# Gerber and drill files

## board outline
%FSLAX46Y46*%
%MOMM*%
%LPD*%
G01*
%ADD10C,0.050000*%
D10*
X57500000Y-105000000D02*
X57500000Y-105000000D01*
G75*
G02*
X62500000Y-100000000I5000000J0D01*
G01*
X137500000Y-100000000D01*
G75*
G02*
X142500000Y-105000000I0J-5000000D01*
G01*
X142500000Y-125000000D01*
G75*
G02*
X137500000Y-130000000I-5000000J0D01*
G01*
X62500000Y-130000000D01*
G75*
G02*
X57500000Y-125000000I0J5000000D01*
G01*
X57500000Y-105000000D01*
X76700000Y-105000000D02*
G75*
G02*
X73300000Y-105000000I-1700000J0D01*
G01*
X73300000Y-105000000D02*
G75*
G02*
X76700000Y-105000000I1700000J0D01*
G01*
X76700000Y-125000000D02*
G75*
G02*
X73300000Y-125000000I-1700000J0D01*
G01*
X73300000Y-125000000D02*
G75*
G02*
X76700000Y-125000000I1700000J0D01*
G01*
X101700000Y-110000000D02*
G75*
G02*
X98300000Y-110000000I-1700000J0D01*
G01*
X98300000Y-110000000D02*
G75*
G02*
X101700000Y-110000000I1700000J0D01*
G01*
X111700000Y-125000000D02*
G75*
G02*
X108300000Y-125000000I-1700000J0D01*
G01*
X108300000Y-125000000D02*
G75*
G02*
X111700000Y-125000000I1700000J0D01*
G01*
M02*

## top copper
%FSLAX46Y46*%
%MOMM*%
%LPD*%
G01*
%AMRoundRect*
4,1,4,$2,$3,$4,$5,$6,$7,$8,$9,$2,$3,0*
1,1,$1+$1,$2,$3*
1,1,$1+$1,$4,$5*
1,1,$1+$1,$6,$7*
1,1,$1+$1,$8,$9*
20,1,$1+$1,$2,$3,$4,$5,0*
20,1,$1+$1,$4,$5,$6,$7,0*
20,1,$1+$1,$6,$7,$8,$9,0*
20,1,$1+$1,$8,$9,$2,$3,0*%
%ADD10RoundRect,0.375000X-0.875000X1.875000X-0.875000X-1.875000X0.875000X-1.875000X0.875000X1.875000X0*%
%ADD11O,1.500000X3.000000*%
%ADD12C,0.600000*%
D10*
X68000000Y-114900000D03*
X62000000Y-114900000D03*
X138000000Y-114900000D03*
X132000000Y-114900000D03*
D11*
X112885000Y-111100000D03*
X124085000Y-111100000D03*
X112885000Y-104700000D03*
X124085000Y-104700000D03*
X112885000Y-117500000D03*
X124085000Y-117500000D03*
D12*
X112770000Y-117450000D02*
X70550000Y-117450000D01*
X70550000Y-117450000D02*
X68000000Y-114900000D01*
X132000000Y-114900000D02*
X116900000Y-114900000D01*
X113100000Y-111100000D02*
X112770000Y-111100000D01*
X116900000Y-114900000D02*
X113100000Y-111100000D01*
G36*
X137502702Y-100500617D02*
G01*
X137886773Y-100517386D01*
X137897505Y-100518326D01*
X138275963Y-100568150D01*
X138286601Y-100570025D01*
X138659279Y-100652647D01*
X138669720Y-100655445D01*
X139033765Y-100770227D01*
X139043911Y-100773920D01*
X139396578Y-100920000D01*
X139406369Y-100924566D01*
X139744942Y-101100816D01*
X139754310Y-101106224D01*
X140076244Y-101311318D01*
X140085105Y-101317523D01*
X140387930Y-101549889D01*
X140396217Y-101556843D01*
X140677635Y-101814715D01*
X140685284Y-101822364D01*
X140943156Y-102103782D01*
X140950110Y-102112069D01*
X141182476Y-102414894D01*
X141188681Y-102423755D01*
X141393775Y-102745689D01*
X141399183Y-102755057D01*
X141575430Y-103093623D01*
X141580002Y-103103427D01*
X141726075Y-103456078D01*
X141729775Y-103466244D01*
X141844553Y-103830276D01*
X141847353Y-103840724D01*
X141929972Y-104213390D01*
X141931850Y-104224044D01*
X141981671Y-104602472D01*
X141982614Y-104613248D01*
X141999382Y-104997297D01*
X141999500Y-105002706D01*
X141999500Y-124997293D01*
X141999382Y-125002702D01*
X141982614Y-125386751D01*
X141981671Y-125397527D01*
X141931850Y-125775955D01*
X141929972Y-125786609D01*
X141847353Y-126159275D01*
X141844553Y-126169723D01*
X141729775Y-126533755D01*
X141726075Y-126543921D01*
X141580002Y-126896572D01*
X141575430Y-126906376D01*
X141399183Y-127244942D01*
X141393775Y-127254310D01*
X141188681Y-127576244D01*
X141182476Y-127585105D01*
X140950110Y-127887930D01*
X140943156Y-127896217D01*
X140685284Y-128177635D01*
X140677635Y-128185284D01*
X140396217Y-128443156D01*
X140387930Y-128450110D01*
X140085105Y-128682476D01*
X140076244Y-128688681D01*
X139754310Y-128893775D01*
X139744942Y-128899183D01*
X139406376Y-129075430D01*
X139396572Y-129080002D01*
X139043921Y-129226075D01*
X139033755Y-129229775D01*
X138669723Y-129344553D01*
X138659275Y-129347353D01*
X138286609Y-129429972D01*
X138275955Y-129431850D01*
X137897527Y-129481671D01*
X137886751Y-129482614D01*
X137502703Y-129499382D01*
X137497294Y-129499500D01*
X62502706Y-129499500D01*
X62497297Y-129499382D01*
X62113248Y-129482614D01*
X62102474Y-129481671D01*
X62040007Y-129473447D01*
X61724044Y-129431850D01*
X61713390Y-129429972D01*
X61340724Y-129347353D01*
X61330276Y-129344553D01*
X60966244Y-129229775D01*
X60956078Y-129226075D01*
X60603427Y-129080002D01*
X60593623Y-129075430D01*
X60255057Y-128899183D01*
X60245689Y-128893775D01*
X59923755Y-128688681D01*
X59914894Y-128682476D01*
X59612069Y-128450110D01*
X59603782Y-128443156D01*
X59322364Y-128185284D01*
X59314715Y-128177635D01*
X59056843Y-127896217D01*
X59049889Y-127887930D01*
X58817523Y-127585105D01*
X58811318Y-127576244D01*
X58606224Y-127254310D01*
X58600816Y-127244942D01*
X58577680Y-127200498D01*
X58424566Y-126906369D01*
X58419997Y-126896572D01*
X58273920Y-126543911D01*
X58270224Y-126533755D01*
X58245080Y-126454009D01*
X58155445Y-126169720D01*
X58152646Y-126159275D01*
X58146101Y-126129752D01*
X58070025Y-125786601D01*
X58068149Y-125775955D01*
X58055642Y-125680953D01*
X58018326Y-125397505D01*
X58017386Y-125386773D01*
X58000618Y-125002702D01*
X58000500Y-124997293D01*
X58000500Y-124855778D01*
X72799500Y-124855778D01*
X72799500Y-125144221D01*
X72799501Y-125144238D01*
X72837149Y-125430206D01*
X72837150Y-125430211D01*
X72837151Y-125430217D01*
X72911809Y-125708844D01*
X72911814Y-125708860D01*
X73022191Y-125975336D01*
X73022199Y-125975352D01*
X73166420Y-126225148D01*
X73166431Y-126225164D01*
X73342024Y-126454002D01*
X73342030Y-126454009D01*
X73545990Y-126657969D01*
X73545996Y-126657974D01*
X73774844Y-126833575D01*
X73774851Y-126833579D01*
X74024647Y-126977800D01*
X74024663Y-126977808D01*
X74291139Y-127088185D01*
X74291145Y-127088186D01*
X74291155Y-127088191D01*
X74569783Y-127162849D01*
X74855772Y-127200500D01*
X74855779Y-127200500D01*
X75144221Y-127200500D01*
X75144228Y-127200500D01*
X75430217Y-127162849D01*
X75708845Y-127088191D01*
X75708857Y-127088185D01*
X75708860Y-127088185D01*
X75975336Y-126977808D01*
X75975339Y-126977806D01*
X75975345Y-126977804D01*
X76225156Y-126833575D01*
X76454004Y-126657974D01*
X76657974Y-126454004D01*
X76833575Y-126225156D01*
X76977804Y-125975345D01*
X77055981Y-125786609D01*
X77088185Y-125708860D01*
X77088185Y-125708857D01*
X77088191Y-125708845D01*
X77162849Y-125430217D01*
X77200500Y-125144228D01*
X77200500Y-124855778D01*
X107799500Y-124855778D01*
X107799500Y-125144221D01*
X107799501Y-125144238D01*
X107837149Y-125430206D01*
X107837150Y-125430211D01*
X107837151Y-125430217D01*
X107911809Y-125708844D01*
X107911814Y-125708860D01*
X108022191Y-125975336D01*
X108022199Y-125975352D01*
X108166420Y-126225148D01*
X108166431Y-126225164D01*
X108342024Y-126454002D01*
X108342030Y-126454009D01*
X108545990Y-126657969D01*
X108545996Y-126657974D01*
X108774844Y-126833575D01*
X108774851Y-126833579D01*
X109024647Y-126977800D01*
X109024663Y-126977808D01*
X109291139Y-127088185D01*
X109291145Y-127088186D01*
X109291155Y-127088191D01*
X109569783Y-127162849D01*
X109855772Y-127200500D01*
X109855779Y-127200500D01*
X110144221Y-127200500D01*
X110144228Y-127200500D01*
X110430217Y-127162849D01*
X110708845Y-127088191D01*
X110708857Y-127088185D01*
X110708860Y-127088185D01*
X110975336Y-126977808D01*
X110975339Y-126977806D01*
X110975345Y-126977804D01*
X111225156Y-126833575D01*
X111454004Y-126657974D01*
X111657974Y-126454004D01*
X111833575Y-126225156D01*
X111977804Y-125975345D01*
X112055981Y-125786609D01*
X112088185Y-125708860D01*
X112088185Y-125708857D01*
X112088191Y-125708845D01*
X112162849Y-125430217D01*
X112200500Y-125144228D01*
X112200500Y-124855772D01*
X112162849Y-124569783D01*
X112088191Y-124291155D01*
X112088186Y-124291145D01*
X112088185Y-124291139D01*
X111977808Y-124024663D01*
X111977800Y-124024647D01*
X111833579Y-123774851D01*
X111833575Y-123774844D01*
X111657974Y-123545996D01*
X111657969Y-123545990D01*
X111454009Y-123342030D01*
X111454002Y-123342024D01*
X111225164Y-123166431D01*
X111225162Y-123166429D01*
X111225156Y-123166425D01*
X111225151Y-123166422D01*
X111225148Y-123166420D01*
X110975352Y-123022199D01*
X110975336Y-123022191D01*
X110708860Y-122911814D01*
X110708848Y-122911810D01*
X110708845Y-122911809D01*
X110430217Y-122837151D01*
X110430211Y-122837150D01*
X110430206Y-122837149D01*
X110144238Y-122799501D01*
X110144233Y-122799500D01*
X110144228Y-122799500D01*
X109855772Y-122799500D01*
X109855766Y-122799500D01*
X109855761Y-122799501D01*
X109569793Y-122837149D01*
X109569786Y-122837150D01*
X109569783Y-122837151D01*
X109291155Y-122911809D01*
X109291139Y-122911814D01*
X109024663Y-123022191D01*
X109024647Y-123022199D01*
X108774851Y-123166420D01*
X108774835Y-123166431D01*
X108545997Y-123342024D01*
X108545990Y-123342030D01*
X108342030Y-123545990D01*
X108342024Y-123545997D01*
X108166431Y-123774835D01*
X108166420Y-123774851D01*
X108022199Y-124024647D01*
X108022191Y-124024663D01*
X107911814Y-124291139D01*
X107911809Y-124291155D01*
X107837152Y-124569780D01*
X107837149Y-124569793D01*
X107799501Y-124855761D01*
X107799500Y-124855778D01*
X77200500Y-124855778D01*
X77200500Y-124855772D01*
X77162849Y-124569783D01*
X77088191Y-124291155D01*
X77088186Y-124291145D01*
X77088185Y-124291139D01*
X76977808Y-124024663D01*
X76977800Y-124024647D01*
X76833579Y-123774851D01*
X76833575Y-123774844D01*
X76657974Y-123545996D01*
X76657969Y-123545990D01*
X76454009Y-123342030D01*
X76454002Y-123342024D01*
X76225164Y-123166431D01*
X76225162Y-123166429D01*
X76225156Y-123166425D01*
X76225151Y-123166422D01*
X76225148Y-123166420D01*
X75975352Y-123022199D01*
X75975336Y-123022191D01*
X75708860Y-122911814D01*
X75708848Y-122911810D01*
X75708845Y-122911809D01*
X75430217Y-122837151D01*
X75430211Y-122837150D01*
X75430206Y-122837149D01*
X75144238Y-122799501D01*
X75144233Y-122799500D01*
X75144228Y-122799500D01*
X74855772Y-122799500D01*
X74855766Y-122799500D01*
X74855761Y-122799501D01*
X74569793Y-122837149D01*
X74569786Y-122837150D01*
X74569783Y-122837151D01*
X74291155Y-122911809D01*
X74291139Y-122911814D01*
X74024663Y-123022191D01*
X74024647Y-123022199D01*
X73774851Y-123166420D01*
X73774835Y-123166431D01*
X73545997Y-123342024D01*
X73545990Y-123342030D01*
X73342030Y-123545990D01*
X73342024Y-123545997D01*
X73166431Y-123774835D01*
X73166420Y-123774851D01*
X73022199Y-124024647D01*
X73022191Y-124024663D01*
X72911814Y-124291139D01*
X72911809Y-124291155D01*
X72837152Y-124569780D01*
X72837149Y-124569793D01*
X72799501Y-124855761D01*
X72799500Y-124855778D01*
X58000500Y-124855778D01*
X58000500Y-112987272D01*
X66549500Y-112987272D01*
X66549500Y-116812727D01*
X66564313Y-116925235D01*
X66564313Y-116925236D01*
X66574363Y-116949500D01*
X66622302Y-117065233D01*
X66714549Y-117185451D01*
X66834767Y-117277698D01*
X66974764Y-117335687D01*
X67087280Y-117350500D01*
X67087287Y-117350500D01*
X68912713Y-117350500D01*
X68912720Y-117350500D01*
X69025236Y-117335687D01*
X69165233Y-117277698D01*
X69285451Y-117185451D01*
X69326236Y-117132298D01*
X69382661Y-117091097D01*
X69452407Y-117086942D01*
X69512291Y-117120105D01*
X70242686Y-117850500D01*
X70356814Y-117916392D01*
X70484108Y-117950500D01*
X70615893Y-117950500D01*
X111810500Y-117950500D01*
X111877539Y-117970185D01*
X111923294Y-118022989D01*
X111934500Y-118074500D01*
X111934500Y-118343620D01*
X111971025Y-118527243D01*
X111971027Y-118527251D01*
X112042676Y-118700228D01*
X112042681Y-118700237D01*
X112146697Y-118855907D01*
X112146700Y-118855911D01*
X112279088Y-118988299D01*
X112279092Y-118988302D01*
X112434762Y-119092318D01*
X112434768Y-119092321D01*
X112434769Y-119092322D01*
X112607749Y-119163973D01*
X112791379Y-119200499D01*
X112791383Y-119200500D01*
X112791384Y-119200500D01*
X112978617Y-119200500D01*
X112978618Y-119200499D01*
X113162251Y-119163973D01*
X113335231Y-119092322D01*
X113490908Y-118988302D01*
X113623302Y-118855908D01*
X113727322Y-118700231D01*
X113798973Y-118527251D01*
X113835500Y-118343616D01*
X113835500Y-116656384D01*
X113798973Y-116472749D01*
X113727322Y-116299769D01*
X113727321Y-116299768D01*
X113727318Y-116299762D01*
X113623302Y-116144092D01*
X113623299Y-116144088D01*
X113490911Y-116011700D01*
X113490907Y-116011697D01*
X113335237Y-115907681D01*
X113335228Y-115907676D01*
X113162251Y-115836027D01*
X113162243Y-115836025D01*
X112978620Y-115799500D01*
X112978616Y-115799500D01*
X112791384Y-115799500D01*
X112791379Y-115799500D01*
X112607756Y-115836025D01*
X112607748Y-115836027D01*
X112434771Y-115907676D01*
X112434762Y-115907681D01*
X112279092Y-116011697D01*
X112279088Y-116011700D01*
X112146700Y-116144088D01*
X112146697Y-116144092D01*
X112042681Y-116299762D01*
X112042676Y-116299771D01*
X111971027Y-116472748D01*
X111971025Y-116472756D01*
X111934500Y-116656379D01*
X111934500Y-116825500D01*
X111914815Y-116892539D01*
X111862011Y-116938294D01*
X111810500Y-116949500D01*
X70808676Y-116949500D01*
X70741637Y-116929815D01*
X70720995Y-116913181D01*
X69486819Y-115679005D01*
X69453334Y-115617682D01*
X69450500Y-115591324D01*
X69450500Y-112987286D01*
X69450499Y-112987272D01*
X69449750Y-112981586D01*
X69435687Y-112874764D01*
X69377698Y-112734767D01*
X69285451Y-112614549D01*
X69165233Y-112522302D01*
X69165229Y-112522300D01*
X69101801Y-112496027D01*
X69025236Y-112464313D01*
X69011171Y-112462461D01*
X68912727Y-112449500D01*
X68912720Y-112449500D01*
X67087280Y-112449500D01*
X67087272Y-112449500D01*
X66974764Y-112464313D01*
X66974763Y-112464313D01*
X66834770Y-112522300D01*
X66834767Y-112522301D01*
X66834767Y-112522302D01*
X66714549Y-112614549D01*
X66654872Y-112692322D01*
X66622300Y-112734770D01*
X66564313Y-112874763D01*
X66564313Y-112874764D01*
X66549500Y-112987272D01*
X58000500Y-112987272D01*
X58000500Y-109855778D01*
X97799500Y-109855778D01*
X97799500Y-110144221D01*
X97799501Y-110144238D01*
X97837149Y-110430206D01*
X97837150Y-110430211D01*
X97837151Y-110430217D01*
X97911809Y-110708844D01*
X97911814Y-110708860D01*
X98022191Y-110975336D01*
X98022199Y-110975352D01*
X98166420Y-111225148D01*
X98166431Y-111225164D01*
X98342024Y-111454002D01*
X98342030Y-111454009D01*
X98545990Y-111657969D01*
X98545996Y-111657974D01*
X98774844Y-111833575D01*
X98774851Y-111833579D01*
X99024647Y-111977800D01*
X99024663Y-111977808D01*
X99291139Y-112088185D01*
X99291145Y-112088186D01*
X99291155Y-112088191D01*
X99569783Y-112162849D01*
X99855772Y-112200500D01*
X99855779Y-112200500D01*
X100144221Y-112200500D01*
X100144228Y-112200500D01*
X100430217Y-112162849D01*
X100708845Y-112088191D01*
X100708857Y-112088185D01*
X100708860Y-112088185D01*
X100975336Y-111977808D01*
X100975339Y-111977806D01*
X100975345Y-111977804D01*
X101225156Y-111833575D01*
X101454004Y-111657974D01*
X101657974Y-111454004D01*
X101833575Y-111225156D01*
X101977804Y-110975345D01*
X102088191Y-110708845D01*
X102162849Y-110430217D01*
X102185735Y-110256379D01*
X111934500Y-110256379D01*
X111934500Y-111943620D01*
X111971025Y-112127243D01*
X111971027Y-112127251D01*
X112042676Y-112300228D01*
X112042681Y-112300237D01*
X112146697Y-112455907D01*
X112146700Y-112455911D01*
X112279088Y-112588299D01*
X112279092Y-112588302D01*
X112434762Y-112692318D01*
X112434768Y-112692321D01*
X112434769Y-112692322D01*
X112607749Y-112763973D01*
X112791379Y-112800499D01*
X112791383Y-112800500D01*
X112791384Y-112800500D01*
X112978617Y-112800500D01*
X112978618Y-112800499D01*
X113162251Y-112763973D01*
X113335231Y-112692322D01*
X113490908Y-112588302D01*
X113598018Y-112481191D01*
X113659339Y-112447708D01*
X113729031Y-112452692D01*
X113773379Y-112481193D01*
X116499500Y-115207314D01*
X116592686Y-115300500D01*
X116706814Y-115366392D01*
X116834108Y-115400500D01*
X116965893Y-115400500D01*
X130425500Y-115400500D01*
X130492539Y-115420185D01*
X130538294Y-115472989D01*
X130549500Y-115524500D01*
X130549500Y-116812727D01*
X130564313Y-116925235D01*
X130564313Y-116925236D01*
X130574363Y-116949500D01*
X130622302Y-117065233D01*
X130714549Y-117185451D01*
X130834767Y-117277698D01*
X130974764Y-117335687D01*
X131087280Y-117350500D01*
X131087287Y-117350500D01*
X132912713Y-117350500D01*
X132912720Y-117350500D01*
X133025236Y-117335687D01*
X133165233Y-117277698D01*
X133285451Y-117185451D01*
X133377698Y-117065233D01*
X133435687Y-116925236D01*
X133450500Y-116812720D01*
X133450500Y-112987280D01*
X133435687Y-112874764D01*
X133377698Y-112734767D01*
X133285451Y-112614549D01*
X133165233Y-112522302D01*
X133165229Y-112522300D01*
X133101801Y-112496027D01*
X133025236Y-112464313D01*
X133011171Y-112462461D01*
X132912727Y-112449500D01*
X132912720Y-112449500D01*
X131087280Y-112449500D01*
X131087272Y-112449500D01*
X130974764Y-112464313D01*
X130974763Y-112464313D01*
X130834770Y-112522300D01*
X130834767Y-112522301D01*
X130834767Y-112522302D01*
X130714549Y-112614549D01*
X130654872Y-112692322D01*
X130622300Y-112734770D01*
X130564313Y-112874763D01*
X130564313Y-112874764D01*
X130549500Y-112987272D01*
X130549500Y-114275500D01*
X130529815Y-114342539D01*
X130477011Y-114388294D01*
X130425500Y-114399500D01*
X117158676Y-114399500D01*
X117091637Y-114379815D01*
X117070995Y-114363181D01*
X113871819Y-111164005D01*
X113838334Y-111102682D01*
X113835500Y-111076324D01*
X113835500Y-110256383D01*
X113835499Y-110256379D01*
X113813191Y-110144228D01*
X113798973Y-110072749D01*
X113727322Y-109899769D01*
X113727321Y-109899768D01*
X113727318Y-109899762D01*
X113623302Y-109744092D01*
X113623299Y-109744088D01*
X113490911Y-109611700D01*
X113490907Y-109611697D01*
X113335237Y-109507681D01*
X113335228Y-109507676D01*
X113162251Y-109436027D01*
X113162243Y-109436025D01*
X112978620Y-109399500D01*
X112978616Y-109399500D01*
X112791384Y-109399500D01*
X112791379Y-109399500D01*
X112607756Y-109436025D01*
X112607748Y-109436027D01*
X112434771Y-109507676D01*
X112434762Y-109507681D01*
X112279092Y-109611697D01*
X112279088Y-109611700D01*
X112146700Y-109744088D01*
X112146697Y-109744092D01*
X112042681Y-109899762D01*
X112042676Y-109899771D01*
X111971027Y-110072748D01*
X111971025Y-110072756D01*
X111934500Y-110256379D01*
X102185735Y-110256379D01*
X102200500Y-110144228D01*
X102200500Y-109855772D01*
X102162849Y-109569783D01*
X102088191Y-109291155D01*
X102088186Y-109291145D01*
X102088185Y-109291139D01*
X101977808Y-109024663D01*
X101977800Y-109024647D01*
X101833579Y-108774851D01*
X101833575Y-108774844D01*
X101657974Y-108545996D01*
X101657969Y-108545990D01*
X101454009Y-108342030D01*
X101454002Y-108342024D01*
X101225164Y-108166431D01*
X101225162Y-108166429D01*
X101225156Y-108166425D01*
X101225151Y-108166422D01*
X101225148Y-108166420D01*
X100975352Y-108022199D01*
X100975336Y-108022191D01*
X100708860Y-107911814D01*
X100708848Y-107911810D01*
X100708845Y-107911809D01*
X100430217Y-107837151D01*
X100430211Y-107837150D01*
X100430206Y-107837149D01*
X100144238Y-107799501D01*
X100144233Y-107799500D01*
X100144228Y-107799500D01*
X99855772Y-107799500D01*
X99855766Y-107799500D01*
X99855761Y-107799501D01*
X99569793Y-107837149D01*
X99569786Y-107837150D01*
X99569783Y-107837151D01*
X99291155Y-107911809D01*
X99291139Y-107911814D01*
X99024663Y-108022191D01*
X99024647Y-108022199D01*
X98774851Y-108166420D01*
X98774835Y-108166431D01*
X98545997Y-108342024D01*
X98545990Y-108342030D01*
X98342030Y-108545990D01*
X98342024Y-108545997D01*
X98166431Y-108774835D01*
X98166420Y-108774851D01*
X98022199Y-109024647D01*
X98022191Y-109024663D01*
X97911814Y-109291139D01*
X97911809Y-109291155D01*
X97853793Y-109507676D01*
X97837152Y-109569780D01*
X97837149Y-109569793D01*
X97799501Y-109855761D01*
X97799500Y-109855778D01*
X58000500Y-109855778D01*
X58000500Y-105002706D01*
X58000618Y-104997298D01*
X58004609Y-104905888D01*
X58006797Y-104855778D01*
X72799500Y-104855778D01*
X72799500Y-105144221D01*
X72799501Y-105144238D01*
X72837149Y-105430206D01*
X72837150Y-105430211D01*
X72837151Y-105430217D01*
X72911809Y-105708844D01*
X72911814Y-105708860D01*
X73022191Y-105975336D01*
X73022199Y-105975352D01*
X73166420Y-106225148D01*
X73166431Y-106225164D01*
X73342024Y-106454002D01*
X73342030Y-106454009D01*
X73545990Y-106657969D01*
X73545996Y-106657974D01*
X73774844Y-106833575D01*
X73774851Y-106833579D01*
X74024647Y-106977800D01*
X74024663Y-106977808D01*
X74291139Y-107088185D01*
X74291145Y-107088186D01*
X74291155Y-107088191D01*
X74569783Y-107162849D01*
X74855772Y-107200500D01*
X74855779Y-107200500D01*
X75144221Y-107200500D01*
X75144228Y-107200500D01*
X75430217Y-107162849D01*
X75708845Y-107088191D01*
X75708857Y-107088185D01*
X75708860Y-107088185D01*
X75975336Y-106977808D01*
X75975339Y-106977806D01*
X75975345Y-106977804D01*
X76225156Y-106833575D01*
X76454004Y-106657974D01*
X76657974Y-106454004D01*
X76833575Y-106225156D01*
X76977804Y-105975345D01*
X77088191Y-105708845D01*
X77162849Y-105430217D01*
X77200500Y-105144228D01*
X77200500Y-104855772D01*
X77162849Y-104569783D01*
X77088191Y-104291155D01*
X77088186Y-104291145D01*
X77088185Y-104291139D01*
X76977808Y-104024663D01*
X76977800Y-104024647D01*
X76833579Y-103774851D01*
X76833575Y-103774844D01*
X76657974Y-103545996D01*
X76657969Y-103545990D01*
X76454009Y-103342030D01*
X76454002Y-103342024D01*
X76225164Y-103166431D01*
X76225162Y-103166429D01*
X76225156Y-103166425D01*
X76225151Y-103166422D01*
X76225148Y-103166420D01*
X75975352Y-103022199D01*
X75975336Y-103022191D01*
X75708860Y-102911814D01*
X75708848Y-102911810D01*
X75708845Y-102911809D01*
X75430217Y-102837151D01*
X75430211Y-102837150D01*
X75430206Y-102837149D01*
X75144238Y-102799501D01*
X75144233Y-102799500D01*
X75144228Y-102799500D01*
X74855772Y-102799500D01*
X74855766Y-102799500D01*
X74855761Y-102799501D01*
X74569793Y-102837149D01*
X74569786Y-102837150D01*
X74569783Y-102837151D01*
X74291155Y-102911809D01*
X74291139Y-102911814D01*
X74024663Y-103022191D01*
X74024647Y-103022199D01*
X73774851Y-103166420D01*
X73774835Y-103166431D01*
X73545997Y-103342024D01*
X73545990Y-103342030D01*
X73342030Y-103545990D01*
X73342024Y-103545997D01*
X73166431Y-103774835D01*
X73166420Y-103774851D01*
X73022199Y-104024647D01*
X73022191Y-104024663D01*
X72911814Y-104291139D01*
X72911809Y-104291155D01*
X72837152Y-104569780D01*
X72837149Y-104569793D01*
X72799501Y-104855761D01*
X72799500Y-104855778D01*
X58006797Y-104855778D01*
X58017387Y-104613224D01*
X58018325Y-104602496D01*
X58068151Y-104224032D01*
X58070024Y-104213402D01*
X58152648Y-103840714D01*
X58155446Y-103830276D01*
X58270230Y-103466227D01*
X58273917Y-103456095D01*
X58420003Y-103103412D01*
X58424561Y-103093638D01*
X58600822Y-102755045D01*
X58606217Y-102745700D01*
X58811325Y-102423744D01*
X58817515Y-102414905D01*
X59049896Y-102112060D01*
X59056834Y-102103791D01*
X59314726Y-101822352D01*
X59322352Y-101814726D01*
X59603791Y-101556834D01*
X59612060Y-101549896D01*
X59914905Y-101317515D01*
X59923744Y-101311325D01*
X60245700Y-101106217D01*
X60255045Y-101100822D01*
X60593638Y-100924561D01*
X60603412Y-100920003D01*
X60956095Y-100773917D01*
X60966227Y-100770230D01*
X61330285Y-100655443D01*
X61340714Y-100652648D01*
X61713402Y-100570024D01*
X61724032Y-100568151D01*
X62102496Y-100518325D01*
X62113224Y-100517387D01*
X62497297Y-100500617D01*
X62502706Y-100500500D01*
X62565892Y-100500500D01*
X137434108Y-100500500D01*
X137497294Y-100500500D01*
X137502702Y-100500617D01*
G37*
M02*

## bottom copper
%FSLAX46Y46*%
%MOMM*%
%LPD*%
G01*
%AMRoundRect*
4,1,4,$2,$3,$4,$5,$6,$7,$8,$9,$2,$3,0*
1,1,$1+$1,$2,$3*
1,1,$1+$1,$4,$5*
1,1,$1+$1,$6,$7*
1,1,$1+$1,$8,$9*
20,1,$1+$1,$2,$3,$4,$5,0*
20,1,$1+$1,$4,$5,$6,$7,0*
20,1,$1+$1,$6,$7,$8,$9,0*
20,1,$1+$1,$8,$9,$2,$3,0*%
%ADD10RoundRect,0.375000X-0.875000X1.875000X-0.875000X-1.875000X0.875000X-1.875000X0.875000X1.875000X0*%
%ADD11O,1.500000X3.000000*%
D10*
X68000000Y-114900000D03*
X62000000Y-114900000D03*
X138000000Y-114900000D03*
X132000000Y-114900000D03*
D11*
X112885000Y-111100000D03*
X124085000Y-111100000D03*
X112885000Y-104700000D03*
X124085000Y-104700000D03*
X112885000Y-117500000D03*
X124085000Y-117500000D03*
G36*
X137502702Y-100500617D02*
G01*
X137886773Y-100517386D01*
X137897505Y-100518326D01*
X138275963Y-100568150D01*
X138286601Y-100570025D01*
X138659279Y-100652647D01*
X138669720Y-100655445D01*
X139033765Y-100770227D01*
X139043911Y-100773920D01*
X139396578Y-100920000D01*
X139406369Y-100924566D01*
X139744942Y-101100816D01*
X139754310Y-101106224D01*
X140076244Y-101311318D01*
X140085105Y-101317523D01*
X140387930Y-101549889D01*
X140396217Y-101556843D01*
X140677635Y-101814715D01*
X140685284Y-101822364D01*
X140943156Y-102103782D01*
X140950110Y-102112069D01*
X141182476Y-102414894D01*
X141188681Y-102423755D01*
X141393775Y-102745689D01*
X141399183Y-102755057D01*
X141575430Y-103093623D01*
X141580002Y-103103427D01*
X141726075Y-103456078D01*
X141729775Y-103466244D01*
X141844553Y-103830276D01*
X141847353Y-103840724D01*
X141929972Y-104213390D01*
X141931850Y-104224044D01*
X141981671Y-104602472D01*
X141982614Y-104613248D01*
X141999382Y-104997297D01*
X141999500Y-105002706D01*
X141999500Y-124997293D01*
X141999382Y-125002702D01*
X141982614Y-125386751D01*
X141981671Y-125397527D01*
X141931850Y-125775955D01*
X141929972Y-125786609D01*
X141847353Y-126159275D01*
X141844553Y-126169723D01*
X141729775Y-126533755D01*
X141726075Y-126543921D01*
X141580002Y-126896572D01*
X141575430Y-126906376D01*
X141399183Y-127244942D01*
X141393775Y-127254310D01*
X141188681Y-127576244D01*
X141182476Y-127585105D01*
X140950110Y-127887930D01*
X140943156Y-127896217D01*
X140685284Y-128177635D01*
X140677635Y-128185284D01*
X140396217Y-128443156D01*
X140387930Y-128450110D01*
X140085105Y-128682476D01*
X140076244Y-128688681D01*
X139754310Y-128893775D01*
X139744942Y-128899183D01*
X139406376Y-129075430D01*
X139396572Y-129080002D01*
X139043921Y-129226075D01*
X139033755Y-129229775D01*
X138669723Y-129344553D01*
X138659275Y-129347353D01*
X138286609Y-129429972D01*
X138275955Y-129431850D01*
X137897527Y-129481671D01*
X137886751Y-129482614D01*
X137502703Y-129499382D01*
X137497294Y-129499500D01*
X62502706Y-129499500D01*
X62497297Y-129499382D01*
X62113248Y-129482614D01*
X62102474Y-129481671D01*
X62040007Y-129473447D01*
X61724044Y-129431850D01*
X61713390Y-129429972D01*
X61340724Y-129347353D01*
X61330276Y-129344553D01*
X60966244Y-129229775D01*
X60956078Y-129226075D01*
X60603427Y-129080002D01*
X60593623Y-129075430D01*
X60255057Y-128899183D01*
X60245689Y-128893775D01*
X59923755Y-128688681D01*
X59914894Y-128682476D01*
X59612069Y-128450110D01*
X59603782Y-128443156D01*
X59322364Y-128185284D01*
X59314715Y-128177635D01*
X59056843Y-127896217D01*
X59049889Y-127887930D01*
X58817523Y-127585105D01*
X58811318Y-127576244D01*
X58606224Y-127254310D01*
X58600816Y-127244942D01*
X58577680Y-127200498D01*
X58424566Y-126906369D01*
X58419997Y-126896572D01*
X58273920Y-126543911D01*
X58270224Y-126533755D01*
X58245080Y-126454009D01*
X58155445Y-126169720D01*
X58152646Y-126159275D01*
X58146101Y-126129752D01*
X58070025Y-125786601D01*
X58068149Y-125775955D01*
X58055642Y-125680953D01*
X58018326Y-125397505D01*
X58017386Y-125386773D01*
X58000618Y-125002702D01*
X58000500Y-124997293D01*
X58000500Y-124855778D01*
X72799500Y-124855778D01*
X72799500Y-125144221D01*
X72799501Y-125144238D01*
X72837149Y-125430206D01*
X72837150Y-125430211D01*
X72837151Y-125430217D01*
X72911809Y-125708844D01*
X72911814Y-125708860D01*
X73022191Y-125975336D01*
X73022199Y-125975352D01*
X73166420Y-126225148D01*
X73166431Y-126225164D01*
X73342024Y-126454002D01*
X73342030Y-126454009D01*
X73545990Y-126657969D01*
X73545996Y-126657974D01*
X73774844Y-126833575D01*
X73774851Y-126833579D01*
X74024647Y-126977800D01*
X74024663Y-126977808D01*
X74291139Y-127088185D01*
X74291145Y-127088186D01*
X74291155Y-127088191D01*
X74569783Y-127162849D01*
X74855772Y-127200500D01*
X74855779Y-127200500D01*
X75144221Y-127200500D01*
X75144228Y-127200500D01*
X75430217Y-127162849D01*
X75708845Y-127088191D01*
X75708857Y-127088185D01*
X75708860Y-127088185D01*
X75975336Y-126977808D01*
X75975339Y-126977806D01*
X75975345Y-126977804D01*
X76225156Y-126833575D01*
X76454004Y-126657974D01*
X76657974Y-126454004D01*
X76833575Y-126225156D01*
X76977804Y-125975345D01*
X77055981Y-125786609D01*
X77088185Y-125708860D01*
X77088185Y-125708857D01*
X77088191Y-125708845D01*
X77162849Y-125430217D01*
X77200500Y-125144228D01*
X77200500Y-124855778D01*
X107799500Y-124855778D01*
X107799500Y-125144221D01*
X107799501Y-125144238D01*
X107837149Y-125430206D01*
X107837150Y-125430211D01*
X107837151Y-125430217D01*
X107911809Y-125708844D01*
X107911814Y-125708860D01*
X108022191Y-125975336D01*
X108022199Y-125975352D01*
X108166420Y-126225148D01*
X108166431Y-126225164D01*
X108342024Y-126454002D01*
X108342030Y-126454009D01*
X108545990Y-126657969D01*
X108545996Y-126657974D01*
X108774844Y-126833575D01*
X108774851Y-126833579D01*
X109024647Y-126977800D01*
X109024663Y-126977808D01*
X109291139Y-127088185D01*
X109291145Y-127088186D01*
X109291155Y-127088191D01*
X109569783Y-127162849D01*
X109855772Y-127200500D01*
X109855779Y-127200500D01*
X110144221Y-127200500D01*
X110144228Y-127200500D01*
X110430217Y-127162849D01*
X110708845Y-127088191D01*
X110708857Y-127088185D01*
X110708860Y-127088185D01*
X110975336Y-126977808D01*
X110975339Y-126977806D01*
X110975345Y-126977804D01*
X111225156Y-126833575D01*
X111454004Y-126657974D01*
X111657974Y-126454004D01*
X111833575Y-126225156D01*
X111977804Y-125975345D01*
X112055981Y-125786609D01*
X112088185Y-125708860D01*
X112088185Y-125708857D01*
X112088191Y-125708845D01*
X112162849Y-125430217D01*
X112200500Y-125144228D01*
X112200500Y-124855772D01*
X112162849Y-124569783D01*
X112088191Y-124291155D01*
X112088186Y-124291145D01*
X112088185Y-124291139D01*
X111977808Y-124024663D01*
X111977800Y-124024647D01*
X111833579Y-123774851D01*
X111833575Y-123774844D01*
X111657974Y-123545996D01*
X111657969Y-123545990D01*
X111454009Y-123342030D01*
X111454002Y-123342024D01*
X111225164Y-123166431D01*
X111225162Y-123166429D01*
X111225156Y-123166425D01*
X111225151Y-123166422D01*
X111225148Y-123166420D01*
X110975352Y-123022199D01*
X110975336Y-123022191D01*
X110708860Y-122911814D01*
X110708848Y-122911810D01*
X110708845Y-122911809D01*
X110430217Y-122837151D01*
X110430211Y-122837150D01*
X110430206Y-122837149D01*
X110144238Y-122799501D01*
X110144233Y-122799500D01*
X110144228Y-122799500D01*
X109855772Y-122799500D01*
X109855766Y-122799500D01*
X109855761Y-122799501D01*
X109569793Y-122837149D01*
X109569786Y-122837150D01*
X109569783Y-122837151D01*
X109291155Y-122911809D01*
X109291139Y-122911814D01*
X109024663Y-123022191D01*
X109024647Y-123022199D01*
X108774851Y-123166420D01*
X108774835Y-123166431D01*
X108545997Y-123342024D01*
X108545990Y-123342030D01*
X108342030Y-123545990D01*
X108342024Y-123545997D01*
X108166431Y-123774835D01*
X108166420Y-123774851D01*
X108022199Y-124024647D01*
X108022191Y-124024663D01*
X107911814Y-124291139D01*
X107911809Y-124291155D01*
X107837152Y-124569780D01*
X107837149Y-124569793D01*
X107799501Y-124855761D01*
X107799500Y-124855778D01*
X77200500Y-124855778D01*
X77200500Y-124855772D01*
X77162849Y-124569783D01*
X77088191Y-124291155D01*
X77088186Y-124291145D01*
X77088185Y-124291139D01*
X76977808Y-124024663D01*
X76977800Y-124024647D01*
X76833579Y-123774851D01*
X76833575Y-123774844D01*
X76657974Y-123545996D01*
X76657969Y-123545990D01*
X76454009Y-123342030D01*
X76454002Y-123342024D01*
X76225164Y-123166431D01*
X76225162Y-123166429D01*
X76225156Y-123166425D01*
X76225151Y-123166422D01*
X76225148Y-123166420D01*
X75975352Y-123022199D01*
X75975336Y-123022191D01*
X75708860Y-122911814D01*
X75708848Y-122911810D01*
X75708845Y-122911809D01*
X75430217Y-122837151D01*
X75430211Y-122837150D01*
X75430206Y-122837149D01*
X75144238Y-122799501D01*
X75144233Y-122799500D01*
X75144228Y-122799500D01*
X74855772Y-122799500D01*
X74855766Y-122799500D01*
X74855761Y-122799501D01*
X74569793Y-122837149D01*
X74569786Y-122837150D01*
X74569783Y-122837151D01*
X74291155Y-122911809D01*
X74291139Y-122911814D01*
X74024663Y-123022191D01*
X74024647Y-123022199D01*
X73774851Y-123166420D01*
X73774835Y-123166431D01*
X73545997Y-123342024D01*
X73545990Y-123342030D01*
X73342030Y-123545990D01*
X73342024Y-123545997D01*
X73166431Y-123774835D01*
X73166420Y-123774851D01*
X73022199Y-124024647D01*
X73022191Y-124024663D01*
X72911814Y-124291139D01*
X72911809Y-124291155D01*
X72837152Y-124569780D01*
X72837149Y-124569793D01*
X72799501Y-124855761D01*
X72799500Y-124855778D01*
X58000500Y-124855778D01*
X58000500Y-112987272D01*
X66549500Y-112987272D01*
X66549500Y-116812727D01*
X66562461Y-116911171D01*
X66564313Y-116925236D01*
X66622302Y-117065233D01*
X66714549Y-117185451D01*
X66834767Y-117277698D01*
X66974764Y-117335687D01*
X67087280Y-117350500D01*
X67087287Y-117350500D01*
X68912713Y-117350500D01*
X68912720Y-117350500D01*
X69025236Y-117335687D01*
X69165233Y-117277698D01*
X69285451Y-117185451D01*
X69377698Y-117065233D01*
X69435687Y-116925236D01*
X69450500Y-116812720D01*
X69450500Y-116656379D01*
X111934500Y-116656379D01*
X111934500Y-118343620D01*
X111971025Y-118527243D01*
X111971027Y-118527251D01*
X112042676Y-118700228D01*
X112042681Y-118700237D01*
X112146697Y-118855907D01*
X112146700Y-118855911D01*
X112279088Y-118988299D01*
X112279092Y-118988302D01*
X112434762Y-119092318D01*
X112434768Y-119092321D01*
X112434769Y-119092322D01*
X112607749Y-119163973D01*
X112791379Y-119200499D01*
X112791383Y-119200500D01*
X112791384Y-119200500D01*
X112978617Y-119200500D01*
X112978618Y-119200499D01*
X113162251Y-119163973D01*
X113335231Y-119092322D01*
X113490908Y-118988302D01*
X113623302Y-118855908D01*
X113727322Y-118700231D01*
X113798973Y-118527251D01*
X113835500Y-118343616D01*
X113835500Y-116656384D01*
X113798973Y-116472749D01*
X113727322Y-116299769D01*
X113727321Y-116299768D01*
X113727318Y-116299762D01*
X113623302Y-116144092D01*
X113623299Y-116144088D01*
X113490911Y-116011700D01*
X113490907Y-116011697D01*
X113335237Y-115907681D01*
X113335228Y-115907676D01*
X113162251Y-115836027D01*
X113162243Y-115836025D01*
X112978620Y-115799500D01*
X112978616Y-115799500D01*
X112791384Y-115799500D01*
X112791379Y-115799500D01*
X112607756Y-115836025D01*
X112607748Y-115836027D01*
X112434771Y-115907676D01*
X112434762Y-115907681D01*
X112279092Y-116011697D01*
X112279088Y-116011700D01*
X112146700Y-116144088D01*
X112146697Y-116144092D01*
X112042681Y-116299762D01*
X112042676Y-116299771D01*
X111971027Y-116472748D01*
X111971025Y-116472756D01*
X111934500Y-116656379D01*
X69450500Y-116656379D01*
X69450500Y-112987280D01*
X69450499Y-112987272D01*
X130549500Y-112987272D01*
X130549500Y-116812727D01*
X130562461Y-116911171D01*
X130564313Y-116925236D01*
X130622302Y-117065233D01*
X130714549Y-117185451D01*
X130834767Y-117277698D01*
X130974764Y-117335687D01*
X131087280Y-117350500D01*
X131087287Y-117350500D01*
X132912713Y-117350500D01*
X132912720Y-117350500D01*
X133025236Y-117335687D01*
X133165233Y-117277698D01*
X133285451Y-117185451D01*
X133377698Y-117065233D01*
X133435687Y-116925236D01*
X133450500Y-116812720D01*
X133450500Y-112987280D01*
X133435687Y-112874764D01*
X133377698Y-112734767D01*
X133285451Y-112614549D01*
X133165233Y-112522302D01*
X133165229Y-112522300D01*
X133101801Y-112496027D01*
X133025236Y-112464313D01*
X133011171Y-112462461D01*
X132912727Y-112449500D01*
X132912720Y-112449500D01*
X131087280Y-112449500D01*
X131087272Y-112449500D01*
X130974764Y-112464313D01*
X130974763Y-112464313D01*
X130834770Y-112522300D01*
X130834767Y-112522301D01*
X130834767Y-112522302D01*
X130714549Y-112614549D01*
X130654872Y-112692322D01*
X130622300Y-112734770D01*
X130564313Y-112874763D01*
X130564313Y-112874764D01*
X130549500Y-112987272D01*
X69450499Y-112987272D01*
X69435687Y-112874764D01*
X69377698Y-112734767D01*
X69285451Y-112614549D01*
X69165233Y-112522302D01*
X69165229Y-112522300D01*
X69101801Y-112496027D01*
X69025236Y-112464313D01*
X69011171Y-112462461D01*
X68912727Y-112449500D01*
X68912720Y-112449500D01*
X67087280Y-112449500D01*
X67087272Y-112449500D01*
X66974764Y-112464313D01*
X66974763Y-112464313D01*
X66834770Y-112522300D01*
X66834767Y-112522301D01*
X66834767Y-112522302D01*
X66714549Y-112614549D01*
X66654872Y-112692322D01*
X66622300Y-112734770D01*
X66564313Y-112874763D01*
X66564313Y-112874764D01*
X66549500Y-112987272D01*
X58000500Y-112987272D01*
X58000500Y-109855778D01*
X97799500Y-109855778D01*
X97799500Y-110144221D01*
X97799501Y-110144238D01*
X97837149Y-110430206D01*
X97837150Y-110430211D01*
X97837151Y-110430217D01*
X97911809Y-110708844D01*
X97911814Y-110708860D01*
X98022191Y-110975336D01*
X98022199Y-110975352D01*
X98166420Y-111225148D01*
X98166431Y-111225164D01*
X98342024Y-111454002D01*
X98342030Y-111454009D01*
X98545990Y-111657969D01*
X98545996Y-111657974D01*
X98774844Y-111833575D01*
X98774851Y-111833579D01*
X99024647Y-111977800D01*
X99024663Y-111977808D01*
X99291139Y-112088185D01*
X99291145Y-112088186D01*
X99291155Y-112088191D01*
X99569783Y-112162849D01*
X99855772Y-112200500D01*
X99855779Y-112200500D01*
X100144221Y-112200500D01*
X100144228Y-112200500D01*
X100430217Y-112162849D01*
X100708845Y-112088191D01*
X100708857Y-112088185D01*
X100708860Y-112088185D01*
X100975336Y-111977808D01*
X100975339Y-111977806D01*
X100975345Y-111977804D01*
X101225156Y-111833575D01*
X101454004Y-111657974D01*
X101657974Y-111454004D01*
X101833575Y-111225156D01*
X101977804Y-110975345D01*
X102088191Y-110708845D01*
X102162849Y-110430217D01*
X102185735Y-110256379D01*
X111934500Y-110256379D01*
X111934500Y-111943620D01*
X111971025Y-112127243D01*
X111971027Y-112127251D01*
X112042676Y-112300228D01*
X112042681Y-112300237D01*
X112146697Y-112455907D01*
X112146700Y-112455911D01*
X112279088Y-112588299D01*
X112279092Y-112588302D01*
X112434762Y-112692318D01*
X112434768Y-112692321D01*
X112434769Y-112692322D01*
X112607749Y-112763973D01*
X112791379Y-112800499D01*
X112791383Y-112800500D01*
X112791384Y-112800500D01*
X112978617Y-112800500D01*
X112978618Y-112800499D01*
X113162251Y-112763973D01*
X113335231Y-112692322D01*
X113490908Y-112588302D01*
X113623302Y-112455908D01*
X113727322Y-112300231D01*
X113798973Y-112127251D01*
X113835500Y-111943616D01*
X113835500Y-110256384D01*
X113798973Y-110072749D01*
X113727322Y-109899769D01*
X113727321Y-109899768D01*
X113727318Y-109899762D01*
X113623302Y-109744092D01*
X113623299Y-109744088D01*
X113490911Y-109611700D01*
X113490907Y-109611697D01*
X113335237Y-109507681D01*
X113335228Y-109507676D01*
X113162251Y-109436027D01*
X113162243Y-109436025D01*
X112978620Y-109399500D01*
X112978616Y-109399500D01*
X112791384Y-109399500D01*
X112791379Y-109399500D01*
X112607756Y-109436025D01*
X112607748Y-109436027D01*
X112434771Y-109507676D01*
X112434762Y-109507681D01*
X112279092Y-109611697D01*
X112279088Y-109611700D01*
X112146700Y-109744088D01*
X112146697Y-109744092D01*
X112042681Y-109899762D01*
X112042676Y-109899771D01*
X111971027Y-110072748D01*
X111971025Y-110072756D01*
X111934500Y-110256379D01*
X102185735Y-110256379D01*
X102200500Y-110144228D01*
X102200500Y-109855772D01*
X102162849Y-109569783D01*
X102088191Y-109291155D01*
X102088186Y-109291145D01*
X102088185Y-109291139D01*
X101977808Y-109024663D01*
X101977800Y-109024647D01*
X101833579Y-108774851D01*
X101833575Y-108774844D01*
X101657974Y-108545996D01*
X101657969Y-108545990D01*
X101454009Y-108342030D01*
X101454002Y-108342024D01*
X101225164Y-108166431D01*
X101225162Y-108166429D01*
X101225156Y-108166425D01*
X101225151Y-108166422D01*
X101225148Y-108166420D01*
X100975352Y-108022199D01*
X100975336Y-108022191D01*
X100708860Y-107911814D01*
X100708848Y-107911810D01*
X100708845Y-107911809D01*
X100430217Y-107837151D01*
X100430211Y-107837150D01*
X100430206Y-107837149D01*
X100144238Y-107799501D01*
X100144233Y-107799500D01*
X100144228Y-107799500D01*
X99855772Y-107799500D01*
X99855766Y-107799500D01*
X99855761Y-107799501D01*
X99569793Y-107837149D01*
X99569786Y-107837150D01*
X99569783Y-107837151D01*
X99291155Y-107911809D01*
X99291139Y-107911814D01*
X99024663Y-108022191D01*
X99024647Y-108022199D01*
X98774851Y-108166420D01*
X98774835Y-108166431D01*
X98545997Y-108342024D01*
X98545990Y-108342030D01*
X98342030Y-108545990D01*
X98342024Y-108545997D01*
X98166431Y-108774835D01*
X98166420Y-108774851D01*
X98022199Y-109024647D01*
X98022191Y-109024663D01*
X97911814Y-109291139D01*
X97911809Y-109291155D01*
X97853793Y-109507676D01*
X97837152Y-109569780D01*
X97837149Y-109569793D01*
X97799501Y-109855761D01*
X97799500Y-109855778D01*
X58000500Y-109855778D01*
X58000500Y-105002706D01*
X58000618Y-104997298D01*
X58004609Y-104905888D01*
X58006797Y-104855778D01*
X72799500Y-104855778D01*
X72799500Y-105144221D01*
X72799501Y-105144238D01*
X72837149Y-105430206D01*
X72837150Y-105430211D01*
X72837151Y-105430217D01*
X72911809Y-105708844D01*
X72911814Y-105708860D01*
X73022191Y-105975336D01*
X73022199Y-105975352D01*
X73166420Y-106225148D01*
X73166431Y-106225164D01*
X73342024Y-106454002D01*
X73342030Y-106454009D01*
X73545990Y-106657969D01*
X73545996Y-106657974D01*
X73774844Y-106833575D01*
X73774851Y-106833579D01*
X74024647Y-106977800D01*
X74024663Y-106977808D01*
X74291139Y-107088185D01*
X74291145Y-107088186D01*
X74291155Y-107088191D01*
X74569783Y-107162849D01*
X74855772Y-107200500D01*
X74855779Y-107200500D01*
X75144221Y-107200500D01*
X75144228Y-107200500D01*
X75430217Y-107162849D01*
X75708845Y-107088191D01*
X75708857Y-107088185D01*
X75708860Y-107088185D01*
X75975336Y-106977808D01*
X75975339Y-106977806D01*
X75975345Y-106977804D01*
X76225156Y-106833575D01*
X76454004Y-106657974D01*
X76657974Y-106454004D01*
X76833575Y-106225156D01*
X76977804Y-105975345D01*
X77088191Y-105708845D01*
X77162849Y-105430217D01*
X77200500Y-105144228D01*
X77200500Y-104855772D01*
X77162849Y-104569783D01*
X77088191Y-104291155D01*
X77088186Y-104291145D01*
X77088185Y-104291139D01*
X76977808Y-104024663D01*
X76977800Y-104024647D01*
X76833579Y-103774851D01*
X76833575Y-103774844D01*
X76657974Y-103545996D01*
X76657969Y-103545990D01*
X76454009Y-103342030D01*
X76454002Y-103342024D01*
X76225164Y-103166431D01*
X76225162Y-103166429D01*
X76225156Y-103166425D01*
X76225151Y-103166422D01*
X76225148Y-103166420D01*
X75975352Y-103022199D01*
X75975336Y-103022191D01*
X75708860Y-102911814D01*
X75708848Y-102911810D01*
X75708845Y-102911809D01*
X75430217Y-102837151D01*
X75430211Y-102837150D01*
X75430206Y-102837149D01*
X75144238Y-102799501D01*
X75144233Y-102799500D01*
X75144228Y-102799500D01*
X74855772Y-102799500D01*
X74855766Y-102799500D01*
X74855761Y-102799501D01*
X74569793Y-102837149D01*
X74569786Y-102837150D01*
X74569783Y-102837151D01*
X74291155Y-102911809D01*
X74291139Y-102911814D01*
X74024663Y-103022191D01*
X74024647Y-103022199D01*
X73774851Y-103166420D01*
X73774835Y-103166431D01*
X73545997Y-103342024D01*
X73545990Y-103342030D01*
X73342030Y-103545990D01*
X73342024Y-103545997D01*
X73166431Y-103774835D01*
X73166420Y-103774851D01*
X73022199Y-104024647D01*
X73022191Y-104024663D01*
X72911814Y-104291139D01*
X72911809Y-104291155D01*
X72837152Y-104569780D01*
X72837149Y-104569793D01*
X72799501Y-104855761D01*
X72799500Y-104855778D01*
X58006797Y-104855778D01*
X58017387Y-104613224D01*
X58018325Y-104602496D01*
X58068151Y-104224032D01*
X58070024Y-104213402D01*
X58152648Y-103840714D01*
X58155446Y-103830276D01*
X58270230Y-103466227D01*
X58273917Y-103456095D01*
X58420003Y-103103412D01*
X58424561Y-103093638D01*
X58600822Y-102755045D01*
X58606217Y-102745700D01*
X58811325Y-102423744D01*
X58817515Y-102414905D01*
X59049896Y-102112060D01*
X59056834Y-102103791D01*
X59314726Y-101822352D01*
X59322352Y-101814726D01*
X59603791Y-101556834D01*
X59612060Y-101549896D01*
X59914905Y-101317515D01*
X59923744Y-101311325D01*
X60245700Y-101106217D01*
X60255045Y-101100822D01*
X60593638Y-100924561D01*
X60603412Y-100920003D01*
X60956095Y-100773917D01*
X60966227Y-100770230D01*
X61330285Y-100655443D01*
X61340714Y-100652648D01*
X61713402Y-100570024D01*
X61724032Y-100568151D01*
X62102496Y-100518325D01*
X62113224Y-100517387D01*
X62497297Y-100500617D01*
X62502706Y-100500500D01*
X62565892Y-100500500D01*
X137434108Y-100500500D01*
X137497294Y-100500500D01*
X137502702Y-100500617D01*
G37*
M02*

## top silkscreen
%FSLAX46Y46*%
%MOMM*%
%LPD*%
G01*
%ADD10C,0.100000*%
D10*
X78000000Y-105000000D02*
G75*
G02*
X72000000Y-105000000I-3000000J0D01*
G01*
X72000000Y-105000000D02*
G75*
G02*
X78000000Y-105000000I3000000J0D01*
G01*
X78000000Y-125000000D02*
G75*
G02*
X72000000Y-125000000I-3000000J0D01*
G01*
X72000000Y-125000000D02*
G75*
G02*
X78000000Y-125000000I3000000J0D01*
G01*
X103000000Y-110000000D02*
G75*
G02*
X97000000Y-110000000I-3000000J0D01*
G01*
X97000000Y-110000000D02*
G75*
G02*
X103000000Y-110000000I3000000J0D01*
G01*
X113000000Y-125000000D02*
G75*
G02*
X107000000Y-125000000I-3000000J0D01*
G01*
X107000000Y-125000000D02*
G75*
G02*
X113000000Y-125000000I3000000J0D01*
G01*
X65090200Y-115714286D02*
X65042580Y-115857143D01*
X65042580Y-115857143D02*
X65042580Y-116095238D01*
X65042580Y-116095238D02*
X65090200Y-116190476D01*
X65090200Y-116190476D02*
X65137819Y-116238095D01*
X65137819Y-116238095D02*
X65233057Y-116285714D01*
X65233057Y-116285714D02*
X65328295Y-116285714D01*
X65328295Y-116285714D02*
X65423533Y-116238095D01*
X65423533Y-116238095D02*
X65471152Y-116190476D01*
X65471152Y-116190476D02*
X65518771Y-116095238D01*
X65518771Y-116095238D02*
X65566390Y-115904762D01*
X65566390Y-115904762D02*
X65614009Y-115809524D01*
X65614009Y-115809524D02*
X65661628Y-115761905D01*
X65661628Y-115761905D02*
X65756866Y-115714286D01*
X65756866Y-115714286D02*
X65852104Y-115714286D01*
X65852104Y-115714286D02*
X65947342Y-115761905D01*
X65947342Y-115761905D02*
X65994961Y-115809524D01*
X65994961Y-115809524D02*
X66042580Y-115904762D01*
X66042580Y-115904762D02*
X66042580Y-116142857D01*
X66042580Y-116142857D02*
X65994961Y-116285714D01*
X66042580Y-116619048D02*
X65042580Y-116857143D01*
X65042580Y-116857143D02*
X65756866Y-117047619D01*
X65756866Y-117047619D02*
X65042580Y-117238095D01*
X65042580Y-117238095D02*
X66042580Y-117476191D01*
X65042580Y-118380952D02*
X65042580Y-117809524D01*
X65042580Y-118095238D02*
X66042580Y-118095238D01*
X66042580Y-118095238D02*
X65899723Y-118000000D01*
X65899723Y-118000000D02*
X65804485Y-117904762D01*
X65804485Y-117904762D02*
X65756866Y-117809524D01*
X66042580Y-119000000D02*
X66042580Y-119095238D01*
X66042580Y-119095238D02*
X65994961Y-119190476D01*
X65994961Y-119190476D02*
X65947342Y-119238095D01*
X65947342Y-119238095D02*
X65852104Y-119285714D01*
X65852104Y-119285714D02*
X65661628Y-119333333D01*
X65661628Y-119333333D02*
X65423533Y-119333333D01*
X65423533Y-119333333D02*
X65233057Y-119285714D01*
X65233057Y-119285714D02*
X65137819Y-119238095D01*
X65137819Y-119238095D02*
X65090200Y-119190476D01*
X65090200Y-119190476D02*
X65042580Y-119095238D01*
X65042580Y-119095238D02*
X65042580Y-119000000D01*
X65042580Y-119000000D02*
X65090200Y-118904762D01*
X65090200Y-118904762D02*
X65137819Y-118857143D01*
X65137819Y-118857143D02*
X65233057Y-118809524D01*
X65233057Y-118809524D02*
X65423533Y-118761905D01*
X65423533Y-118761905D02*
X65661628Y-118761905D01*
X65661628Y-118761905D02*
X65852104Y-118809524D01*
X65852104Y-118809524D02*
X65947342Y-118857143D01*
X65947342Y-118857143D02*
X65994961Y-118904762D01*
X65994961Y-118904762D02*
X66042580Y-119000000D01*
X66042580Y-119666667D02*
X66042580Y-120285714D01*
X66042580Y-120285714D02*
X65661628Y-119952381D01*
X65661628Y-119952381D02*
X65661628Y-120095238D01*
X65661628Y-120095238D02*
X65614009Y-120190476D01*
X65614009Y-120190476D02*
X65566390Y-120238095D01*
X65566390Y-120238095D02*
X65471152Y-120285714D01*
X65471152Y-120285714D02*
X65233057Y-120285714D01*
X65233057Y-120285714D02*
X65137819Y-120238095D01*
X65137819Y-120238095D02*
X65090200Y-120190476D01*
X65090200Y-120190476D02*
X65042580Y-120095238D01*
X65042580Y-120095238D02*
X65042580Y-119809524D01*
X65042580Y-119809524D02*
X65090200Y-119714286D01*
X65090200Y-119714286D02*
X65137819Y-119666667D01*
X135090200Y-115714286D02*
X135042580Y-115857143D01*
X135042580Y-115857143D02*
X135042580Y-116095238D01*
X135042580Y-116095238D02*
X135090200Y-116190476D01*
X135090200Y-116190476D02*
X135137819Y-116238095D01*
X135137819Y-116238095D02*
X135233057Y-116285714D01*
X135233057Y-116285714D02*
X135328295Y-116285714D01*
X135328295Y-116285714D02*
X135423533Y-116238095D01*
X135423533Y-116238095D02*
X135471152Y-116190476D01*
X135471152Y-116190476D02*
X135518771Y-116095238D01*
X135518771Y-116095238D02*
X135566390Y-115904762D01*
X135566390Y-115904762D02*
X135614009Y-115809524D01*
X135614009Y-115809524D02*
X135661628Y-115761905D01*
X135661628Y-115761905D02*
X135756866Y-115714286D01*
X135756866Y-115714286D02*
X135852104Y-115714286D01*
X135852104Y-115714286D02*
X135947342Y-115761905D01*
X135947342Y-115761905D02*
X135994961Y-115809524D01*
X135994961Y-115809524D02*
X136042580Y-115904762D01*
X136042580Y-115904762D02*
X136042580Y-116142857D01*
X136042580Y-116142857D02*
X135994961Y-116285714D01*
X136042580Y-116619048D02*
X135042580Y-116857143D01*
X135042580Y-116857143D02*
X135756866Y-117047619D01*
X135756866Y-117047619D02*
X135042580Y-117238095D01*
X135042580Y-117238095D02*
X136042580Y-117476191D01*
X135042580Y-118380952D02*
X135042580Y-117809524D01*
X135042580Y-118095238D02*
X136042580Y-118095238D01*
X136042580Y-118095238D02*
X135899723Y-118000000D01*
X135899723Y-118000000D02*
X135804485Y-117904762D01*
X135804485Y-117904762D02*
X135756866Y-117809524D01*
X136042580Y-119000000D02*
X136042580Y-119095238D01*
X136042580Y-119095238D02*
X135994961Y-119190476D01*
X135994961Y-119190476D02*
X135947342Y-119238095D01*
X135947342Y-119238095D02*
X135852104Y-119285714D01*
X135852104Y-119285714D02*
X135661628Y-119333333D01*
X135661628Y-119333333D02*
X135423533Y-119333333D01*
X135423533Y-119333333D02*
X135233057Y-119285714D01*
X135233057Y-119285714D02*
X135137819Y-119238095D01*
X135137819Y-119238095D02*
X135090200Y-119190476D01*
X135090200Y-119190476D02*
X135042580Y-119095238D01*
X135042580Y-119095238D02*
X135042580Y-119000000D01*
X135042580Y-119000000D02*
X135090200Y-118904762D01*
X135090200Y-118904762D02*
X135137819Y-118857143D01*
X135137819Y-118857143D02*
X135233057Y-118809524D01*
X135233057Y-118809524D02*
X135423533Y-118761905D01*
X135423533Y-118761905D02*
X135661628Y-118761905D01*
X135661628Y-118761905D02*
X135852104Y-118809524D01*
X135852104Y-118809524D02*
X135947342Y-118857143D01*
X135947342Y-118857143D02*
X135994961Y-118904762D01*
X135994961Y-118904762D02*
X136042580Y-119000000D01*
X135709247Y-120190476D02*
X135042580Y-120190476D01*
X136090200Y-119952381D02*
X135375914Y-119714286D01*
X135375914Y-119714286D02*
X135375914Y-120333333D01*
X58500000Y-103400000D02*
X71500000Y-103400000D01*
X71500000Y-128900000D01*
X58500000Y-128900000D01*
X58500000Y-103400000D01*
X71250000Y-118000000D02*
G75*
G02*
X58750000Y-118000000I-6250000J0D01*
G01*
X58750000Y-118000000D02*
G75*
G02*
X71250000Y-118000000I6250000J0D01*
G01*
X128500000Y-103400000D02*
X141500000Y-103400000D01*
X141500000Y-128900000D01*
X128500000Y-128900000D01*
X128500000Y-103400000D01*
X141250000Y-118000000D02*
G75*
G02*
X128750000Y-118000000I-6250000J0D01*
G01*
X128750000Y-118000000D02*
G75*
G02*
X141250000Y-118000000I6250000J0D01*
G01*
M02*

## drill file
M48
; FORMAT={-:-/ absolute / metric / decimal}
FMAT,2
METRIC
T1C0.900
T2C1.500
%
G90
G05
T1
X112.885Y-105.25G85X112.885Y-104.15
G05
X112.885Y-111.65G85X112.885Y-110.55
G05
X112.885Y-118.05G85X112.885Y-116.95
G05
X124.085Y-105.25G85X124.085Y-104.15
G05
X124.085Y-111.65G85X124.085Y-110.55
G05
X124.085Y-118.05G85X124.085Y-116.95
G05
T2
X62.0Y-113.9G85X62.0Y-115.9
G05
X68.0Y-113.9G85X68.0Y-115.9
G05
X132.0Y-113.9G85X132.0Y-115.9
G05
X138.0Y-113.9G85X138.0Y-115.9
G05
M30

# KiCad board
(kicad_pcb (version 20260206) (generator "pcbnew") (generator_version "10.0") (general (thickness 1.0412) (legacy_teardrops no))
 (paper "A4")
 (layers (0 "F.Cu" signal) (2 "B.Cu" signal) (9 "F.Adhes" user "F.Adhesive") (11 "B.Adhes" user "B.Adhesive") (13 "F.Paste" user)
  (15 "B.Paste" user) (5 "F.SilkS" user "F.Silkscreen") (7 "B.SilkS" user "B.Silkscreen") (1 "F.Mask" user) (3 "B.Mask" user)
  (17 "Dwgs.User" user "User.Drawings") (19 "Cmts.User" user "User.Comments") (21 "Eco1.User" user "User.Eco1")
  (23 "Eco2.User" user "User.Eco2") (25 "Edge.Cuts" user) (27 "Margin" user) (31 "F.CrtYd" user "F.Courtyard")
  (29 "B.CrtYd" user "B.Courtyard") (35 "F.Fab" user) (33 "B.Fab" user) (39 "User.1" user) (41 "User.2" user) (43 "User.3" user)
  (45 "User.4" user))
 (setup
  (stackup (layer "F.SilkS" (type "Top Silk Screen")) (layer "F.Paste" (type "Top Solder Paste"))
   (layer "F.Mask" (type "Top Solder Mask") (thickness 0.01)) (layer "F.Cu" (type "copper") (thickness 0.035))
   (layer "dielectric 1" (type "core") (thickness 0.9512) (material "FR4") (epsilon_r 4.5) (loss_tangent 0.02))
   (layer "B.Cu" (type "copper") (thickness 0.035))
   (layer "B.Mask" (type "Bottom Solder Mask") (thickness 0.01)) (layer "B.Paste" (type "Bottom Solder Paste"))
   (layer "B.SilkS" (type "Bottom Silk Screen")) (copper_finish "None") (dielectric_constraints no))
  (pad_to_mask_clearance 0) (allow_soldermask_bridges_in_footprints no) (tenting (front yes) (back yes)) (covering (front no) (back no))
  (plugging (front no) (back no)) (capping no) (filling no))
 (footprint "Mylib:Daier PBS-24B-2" (layer "F.Cu") (at 65 118 -90)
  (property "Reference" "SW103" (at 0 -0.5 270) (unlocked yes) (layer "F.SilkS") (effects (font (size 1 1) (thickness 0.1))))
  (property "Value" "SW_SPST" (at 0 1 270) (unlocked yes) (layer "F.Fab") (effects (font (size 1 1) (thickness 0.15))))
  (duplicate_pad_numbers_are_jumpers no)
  (fp_rect (start -14.6 -6.5) (end 10.9 6.5) (stroke (width 0.1) (type solid)) (fill no) (layer "F.SilkS"))
  (fp_circle (center 0 0) (end 6.25 0) (stroke (width 0.1) (type solid)) (fill no) (layer "F.SilkS"))
  (pad "1" thru_hole roundrect (at -3.1 -3 270) (size 4.5 2.5) (drill oval 3.5 1.5) (layers "*.Cu" "*.Mask") (remove_unused_layers no)
   (roundrect_rratio 0.15) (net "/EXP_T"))
  (pad "2" thru_hole roundrect (at -3.1 3 270) (size 4.5 2.5) (drill oval 3.5 1.5) (layers "*.Cu" "*.Mask") (remove_unused_layers no)
   (roundrect_rratio 0.15) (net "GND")))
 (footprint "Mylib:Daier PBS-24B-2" (layer "F.Cu") (at 135 118 -90)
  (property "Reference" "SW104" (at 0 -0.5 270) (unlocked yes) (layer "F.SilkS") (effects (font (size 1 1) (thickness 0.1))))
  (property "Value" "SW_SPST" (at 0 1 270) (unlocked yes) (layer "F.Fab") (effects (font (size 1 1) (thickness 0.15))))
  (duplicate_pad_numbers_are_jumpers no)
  (fp_rect (start -14.6 -6.5) (end 10.9 6.5) (stroke (width 0.1) (type solid)) (fill no) (layer "F.SilkS"))
  (fp_circle (center 0 0) (end 6.25 0) (stroke (width 0.1) (type solid)) (fill no) (layer "F.SilkS"))
  (pad "1" thru_hole roundrect (at -3.1 -3 270) (size 4.5 2.5) (drill oval 3.5 1.5) (layers "*.Cu" "*.Mask") (remove_unused_layers no)
   (roundrect_rratio 0.15) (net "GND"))
  (pad "2" thru_hole roundrect (at -3.1 3 270) (size 4.5 2.5) (drill oval 3.5 1.5) (layers "*.Cu" "*.Mask") (remove_unused_layers no)
   (roundrect_rratio 0.15) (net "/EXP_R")))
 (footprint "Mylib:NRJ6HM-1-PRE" (layer "F.Cu") (at 120 100 90)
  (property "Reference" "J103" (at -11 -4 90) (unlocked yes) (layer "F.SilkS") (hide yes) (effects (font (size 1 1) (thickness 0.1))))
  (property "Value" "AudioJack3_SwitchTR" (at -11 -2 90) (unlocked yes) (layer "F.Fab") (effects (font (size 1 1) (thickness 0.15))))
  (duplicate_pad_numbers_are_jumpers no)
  (pad "R" thru_hole oval (at -11.1 -7.115 90) (size 3 1.5) (drill oval 2 0.9) (layers "*.Cu" "*.Mask") (remove_unused_layers no)
   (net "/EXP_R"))
  (pad "RN" thru_hole oval (at -11.1 4.085 90) (size 3 1.5) (drill oval 2 0.9) (layers "*.Cu" "*.Mask") (remove_unused_layers no)
   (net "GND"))
  (pad "S" thru_hole oval (at -4.7 -7.115 90) (size 3 1.5) (drill oval 2 0.9) (layers "*.Cu" "*.Mask") (remove_unused_layers no) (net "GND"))
  (pad "S" thru_hole oval (at -4.7 4.085 90) (size 3 1.5) (drill oval 2 0.9) (layers "*.Cu" "*.Mask") (remove_unused_layers no) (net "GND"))
  (pad "T" thru_hole oval (at -17.5 -7.115 90) (size 3 1.5) (drill oval 2 0.9) (layers "*.Cu" "*.Mask") (remove_unused_layers no)
   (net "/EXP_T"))
  (pad "TN" thru_hole oval (at -17.5 4.085 90) (size 3 1.5) (drill oval 2 0.9) (layers "*.Cu" "*.Mask") (remove_unused_layers no)
   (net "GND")))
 (gr_circle (center 75 105) (end 78 105) (stroke (width 0.1) (type default)) (fill no) (layer "F.SilkS"))
 (gr_circle (center 75 125) (end 78 125) (stroke (width 0.1) (type default)) (fill no) (layer "F.SilkS"))
 (gr_circle (center 100 110) (end 103 110) (stroke (width 0.1) (type solid)) (fill no) (layer "F.SilkS"))
 (gr_circle (center 110 125) (end 113 125) (stroke (width 0.1) (type solid)) (fill no) (layer "F.SilkS"))
 (gr_rect (start 57.5 100) (end 142.5 130) (radius 5) (stroke (width 0.05) (type solid)) (fill no) (layer "Edge.Cuts"))
 (gr_circle (center 75 105) (end 76.7 105) (stroke (width 0.05) (type solid)) (fill no) (layer "Edge.Cuts"))
 (gr_circle (center 75 125) (end 76.7 125) (stroke (width 0.05) (type solid)) (fill no) (layer "Edge.Cuts"))
 (gr_circle (center 100 110) (end 101.7 110) (stroke (width 0.05) (type solid)) (fill no) (layer "Edge.Cuts"))
 (gr_circle (center 110 125) (end 111.7 125) (stroke (width 0.05) (type solid)) (fill no) (layer "Edge.Cuts"))
 (segment (start 112.77 117.45) (end 70.55 117.45) (width 0.6) (layer "F.Cu") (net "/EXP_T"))
 (segment (start 70.55 117.45) (end 68 114.9) (width 0.6) (layer "F.Cu") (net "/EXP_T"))
 (segment (start 132 114.9) (end 116.9 114.9) (width 0.6) (layer "F.Cu") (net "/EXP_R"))
 (segment (start 113.1 111.1) (end 112.77 111.1) (width 0.6) (layer "F.Cu") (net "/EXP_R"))
 (segment (start 116.9 114.9) (end 113.1 111.1) (width 0.6) (layer "F.Cu") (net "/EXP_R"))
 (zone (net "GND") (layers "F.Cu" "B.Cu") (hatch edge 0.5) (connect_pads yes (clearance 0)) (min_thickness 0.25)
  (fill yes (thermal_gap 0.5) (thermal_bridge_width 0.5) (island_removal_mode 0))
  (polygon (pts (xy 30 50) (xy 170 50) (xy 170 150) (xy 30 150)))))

